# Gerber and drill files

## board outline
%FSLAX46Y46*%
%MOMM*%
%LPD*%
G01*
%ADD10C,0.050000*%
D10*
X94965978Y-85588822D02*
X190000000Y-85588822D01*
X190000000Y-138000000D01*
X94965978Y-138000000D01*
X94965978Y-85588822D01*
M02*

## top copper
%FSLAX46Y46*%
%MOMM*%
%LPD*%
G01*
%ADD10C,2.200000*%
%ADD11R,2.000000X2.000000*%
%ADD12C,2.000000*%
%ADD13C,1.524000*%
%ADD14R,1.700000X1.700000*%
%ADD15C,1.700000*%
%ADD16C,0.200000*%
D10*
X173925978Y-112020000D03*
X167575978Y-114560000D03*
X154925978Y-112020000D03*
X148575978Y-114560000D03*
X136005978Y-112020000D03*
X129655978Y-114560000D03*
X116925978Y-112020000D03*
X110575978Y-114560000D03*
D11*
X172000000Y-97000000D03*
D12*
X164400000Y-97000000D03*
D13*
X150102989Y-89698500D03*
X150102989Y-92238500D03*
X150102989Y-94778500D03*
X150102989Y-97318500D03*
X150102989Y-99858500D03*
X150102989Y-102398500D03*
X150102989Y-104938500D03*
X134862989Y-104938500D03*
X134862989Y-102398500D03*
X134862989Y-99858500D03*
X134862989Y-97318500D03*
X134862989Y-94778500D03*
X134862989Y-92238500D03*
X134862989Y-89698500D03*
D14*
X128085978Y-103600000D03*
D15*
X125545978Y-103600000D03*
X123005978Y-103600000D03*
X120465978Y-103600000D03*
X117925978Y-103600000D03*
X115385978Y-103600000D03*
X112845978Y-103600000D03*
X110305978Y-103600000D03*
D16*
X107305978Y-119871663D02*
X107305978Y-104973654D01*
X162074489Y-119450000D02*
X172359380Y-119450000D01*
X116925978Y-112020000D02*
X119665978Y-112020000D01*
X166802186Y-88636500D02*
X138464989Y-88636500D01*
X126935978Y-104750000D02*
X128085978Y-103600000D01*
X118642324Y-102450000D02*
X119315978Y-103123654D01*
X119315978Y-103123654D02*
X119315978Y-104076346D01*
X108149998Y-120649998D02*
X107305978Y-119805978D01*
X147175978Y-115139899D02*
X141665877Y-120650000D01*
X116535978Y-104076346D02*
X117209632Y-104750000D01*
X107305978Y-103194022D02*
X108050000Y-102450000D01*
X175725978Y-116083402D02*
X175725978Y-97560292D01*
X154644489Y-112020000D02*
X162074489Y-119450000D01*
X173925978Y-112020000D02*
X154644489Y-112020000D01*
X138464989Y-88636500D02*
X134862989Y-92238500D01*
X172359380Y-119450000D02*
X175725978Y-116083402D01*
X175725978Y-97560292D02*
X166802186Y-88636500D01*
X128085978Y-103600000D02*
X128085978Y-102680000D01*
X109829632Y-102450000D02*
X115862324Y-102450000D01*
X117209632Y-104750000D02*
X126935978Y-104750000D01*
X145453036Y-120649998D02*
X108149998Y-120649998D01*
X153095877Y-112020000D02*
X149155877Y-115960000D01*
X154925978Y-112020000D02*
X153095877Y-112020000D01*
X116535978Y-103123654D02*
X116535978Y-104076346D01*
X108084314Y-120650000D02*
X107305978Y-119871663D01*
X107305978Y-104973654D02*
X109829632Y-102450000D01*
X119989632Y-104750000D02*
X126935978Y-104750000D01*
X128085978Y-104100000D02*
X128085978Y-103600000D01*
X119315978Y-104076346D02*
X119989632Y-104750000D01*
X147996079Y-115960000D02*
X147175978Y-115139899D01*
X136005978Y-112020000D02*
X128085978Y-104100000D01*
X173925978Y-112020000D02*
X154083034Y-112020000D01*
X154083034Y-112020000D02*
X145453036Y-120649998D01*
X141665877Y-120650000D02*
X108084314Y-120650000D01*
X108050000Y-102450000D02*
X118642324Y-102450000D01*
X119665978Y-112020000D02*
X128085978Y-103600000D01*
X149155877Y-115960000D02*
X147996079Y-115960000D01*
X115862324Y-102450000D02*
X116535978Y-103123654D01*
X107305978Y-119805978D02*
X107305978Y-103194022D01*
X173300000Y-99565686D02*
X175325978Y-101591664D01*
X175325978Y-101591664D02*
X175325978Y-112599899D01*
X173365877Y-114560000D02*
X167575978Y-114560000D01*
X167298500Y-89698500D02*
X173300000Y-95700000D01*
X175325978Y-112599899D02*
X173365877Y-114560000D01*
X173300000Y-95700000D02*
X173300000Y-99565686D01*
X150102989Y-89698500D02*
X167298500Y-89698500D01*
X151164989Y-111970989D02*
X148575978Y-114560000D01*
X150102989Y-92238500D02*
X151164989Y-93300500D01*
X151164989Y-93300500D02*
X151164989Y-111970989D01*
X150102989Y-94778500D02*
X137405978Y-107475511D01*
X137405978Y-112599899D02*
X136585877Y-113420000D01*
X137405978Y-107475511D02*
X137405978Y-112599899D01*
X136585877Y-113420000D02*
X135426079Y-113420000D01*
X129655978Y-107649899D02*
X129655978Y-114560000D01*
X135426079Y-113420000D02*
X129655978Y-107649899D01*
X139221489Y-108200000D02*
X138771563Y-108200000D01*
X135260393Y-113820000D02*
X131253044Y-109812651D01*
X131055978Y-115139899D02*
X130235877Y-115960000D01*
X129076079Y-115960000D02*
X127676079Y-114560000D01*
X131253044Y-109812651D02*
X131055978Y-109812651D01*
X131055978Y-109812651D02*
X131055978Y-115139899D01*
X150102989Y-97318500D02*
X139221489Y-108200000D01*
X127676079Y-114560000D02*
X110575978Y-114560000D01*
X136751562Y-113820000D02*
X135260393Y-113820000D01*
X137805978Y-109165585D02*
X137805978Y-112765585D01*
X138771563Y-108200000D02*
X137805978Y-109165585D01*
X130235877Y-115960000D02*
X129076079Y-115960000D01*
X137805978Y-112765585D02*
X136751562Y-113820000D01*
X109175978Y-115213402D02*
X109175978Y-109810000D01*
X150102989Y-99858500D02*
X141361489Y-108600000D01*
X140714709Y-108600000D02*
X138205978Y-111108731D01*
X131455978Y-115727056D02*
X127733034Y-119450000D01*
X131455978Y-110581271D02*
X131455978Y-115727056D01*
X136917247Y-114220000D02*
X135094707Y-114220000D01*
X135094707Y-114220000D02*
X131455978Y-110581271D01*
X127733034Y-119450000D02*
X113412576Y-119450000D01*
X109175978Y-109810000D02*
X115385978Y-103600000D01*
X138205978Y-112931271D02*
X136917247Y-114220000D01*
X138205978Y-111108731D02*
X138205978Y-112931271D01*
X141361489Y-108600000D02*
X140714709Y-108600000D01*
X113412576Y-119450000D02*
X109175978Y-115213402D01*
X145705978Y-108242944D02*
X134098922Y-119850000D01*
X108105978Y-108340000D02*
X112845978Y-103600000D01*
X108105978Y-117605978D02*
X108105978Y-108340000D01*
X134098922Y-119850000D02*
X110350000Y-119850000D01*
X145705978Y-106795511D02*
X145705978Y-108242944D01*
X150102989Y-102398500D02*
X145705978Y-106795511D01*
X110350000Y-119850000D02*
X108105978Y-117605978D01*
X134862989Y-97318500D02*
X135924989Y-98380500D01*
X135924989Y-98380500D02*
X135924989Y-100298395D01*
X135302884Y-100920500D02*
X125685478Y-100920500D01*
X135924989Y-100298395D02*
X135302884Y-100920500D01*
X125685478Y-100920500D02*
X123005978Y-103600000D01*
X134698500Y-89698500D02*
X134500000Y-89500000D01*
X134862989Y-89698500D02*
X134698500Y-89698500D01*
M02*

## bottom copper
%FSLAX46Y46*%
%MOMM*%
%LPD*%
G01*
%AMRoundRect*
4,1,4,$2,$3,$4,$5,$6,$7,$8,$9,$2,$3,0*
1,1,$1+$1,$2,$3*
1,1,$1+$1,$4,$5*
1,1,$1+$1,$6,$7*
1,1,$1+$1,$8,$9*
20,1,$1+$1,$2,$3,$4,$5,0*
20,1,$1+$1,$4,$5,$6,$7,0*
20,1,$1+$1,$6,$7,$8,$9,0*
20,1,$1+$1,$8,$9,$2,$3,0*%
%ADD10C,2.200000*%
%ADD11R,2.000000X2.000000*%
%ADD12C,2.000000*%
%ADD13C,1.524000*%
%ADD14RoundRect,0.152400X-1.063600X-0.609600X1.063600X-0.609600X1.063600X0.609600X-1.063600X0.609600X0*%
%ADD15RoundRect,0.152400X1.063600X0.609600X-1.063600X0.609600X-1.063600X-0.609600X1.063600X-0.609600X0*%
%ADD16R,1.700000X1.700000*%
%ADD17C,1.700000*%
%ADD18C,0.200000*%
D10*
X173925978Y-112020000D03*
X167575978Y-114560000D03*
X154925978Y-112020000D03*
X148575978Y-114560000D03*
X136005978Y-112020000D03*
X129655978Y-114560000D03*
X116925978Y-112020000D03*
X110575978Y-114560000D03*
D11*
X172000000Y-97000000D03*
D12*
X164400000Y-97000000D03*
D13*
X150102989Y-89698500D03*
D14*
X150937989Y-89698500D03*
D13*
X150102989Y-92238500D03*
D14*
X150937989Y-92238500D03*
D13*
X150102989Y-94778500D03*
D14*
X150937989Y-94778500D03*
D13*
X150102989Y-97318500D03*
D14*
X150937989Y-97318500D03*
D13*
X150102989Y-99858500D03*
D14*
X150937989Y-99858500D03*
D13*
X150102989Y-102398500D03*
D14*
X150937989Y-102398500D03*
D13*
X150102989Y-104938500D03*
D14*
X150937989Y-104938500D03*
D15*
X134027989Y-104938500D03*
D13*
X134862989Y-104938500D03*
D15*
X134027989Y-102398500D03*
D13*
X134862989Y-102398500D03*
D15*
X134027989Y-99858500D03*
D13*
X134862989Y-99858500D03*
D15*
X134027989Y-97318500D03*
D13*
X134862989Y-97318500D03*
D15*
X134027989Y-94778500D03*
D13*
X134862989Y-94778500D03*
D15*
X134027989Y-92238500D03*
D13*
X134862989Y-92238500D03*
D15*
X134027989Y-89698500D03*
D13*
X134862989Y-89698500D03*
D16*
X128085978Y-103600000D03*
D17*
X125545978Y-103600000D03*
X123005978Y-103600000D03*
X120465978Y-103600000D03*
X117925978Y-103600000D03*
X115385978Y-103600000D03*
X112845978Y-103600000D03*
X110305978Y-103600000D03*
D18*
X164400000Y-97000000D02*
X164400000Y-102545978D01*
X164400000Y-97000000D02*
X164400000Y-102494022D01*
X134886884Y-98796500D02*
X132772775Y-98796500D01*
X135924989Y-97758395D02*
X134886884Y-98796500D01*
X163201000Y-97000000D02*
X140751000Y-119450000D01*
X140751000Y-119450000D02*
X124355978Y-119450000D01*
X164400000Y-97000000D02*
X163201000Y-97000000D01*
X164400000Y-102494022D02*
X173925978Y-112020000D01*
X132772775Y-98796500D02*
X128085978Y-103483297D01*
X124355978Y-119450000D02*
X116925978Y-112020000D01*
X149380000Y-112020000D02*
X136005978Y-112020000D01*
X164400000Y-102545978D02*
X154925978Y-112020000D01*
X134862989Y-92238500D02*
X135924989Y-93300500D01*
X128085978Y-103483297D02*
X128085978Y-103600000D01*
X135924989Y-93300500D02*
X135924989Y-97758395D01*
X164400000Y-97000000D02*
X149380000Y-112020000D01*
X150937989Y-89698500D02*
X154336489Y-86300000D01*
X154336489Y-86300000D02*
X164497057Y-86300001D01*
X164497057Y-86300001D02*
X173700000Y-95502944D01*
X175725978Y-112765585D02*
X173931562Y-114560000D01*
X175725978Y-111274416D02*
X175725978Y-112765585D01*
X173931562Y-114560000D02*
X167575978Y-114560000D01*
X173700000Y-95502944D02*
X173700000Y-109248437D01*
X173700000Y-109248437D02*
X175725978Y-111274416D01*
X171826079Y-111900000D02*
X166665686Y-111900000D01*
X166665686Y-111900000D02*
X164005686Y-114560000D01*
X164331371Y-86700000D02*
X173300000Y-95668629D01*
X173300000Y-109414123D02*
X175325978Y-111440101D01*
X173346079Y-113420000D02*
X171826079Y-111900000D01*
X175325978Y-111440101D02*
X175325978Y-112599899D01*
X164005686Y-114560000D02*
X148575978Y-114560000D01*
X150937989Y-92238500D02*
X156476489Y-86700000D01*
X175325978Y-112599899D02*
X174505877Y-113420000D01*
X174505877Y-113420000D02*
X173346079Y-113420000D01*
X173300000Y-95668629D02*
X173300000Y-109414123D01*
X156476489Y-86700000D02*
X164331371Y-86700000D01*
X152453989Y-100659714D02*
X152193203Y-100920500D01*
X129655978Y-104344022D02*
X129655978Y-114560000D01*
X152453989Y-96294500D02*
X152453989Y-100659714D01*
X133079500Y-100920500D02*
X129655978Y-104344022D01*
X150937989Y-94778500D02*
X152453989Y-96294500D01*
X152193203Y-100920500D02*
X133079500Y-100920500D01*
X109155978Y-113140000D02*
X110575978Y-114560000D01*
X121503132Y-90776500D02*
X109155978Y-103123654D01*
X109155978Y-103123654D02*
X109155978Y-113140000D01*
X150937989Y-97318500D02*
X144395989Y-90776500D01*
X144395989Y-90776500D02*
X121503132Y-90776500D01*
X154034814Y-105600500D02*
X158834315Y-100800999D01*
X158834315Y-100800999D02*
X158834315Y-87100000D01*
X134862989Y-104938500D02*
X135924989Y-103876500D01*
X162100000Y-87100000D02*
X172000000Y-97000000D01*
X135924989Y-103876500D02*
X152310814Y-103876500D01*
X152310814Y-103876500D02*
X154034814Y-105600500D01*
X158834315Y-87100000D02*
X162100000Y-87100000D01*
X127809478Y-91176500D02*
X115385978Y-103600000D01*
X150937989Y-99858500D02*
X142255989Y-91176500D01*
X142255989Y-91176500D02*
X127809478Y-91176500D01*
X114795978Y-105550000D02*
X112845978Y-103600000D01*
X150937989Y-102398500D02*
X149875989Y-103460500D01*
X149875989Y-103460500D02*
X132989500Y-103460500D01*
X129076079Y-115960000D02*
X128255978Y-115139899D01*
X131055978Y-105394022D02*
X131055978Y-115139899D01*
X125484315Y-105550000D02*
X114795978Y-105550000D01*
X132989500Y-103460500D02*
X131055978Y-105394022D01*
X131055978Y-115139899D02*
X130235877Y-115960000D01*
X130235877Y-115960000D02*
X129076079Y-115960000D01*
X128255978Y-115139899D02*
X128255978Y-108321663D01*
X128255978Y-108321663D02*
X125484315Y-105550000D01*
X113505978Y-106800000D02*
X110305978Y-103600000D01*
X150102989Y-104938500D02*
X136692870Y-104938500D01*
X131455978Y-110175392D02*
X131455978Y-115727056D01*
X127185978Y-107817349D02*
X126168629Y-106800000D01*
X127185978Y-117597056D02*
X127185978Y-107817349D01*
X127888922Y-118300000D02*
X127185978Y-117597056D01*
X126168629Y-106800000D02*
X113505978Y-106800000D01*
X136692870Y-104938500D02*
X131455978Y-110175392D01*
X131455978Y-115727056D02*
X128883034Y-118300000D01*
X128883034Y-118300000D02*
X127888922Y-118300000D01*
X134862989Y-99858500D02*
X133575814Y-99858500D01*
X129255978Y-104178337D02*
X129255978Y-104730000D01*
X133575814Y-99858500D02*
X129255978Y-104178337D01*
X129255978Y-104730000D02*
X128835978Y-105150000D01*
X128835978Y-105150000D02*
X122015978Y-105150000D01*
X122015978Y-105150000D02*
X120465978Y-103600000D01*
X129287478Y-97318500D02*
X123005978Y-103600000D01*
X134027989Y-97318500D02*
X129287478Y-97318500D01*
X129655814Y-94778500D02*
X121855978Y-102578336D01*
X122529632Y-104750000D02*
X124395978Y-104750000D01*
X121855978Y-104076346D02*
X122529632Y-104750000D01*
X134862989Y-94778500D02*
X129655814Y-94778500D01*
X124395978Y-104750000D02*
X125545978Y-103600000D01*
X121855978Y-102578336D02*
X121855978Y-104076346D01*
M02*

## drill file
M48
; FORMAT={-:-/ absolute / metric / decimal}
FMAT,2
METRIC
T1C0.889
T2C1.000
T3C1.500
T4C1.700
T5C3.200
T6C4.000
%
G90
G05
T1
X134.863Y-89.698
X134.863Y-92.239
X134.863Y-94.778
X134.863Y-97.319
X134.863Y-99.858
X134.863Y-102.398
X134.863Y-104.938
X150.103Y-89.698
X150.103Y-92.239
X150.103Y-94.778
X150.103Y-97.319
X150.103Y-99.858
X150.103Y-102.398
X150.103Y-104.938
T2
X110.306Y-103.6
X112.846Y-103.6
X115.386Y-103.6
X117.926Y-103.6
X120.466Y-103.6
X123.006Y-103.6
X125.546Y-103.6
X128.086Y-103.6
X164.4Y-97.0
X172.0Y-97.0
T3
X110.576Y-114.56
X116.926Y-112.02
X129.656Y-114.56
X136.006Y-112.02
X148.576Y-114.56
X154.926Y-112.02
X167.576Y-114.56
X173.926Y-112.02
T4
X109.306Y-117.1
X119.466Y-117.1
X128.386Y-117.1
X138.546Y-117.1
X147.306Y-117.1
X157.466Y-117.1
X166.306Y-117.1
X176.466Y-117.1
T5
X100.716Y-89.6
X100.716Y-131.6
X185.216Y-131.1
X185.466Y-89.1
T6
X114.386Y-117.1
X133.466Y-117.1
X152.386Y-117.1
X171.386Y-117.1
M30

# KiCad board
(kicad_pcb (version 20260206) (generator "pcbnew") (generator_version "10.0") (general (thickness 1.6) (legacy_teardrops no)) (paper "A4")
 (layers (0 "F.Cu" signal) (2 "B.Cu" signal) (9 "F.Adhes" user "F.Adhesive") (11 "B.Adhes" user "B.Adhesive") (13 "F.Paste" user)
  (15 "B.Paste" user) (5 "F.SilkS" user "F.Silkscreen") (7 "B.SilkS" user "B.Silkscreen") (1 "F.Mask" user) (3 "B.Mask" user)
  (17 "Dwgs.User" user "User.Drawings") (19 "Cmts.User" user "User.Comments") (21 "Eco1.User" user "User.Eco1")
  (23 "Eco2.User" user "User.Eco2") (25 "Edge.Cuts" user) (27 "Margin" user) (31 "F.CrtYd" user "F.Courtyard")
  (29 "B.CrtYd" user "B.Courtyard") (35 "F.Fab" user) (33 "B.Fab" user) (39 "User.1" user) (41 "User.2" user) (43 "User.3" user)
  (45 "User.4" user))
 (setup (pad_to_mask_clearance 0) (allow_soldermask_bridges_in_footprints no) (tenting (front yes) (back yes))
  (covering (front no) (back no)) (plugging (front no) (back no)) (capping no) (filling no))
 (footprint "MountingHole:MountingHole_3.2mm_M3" (layer "F.Cu") (at 185.215978 131.1)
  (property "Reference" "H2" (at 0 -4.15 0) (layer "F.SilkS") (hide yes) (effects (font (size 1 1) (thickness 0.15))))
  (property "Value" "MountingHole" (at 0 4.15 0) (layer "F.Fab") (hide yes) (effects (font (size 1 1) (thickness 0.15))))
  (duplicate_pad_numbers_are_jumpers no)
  (pad "" np_thru_hole circle (at 0 0) (size 3.2 3.2) (drill 3.2) (layers "*.Cu" "*.Mask")))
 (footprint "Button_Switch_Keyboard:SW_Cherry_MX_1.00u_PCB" (layer "F.Cu") (at 173.925978 112.02)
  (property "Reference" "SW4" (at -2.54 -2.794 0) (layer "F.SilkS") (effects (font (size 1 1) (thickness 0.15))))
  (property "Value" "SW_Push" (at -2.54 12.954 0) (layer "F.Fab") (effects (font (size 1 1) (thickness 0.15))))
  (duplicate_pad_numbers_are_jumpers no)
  (pad "" np_thru_hole circle (at -7.62 5.08) (size 1.7 1.7) (drill 1.7) (layers "*.Cu" "*.Mask"))
  (pad "" np_thru_hole circle (at -2.54 5.08) (size 4 4) (drill 4) (layers "*.Cu" "*.Mask"))
  (pad "" np_thru_hole circle (at 2.54 5.08) (size 1.7 1.7) (drill 1.7) (layers "*.Cu" "*.Mask"))
  (pad "1" thru_hole circle (at 0 0) (size 2.2 2.2) (drill 1.5) (layers "*.Cu" "*.Mask") (remove_unused_layers no) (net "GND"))
  (pad "2" thru_hole circle (at -6.35 2.54) (size 2.2 2.2) (drill 1.5) (layers "*.Cu" "*.Mask") (remove_unused_layers no)
   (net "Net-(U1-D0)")))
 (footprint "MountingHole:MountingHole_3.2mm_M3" (layer "F.Cu") (at 100.715978 131.6)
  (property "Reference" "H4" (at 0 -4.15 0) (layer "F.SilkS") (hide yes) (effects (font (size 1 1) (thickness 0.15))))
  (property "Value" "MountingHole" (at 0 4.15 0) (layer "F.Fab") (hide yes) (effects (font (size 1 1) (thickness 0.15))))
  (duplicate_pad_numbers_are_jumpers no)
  (pad "" np_thru_hole circle (at 0 0) (size 3.2 3.2) (drill 3.2) (layers "*.Cu" "*.Mask")))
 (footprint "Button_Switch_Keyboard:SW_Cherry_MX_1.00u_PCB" (layer "F.Cu") (at 154.925978 112.02)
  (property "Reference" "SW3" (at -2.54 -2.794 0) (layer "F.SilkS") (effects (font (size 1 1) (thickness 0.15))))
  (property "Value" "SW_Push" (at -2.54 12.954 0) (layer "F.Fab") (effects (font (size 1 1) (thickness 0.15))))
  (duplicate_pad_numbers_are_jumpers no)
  (pad "" np_thru_hole circle (at -7.62 5.08) (size 1.7 1.7) (drill 1.7) (layers "*.Cu" "*.Mask"))
  (pad "" np_thru_hole circle (at -2.54 5.08) (size 4 4) (drill 4) (layers "*.Cu" "*.Mask"))
  (pad "" np_thru_hole circle (at 2.54 5.08) (size 1.7 1.7) (drill 1.7) (layers "*.Cu" "*.Mask"))
  (pad "1" thru_hole circle (at 0 0) (size 2.2 2.2) (drill 1.5) (layers "*.Cu" "*.Mask") (remove_unused_layers no) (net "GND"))
  (pad "2" thru_hole circle (at -6.35 2.54) (size 2.2 2.2) (drill 1.5) (layers "*.Cu" "*.Mask") (remove_unused_layers no)
   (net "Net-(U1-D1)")))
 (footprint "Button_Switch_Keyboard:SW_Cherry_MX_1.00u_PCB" (layer "F.Cu") (at 136.005978 112.02)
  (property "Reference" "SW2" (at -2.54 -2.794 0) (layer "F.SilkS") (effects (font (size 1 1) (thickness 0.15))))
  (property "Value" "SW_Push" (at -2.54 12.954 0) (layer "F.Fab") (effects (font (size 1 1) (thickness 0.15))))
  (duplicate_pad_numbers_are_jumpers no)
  (pad "" np_thru_hole circle (at -7.62 5.08) (size 1.7 1.7) (drill 1.7) (layers "*.Cu" "*.Mask"))
  (pad "" np_thru_hole circle (at -2.54 5.08) (size 4 4) (drill 4) (layers "*.Cu" "*.Mask"))
  (pad "" np_thru_hole circle (at 2.54 5.08) (size 1.7 1.7) (drill 1.7) (layers "*.Cu" "*.Mask"))
  (pad "1" thru_hole circle (at 0 0) (size 2.2 2.2) (drill 1.5) (layers "*.Cu" "*.Mask") (remove_unused_layers no) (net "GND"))
  (pad "2" thru_hole circle (at -6.35 2.54) (size 2.2 2.2) (drill 1.5) (layers "*.Cu" "*.Mask") (remove_unused_layers no)
   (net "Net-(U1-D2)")))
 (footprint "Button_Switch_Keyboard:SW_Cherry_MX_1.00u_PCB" (layer "F.Cu") (at 116.925978 112.02)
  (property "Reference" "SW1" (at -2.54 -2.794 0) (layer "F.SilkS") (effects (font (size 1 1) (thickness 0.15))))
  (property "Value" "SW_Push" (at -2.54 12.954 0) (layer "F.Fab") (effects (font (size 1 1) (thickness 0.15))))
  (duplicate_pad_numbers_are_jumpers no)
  (pad "" np_thru_hole circle (at -7.62 5.08) (size 1.7 1.7) (drill 1.7) (layers "*.Cu" "*.Mask"))
  (pad "" np_thru_hole circle (at -2.54 5.08) (size 4 4) (drill 4) (layers "*.Cu" "*.Mask"))
  (pad "" np_thru_hole circle (at 2.54 5.08) (size 1.7 1.7) (drill 1.7) (layers "*.Cu" "*.Mask"))
  (pad "1" thru_hole circle (at 0 0) (size 2.2 2.2) (drill 1.5) (layers "*.Cu" "*.Mask") (remove_unused_layers no) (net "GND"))
  (pad "2" thru_hole circle (at -6.35 2.54) (size 2.2 2.2) (drill 1.5) (layers "*.Cu" "*.Mask") (remove_unused_layers no)
   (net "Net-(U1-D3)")))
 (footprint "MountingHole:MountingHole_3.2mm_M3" (layer "F.Cu") (at 100.715978 89.6)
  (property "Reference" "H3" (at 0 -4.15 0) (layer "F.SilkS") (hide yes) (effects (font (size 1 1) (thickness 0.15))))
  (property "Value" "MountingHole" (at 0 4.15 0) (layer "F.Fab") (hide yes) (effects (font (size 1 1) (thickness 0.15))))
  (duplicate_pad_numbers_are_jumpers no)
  (pad "" np_thru_hole circle (at 0 0) (size 3.2 3.2) (drill 3.2) (layers "*.Cu" "*.Mask")))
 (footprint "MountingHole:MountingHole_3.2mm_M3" (layer "F.Cu") (at 185.465978 89.1)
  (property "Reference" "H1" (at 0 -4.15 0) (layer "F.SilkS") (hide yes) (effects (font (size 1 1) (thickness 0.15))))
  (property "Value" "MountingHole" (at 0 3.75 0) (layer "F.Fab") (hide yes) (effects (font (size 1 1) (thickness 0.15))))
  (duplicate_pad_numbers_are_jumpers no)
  (pad "" np_thru_hole circle (at 0 0) (size 3.2 3.2) (drill 3.2) (layers "*.Cu" "*.Mask")))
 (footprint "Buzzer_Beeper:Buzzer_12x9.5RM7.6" (layer "B.Cu") (at 172 97 180)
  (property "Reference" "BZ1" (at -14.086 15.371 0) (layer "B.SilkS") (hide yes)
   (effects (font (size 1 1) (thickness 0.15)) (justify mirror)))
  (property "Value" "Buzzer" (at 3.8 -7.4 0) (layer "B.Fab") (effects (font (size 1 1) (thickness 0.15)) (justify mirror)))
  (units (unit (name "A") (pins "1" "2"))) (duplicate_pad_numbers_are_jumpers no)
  (pad "1" thru_hole rect (at 0 0 180) (size 2 2) (drill 1) (layers "*.Cu" "*.Mask") (remove_unused_layers no) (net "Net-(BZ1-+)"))
  (pad "2" thru_hole circle (at 7.6 0 180) (size 2 2) (drill 1) (layers "*.Cu" "*.Mask") (remove_unused_layers no) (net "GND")))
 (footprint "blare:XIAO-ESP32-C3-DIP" (layer "B.Cu") (at 142.482989 97.3185 90)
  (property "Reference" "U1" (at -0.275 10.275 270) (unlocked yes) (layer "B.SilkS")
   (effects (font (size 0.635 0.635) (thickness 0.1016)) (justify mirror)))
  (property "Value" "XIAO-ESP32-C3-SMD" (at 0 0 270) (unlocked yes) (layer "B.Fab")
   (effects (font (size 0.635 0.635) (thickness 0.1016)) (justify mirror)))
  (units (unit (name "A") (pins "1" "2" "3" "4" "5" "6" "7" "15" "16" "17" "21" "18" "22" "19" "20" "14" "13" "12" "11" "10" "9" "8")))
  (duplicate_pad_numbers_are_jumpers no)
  (pad "1" thru_hole circle (at 7.62 7.62) (size 1.524 1.524) (drill 0.889) (layers "*.Cu" "*.Mask") (remove_unused_layers no)
   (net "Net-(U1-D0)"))
  (pad "1" smd roundrect (at 7.62 8.455) (size 2.432 1.524) (layers "B.Cu" "B.Mask") (roundrect_rratio 0.1) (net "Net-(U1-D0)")
   (thermal_bridge_angle 45))
  (pad "2" thru_hole circle (at 5.08 7.62) (size 1.524 1.524) (drill 0.889) (layers "*.Cu" "*.Mask") (remove_unused_layers no)
   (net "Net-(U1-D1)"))
  (pad "2" smd roundrect (at 5.08 8.455) (size 2.432 1.524) (layers "B.Cu" "B.Mask") (roundrect_rratio 0.1) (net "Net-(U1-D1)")
   (thermal_bridge_angle 45))
  (pad "3" thru_hole circle (at 2.54 7.62) (size 1.524 1.524) (drill 0.889) (layers "*.Cu" "*.Mask") (remove_unused_layers no)
   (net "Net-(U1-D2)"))
  (pad "3" smd roundrect (at 2.54 8.455) (size 2.432 1.524) (layers "B.Cu" "B.Mask") (roundrect_rratio 0.1) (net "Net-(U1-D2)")
   (thermal_bridge_angle 45))
  (pad "4" thru_hole circle (at 0 7.62) (size 1.524 1.524) (drill 0.889) (layers "*.Cu" "*.Mask") (remove_unused_layers no)
   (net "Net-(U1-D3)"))
  (pad "4" smd roundrect (at 0 8.455) (size 2.432 1.524) (layers "B.Cu" "B.Mask") (roundrect_rratio 0.1) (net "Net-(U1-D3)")
   (thermal_bridge_angle 45))
  (pad "5" thru_hole circle (at -2.54 7.62) (size 1.524 1.524) (drill 0.889) (layers "*.Cu" "*.Mask") (remove_unused_layers no) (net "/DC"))
  (pad "5" smd roundrect (at -2.54 8.455) (size 2.432 1.524) (layers "B.Cu" "B.Mask") (roundrect_rratio 0.1) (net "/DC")
   (thermal_bridge_angle 45))
  (pad "6" thru_hole circle (at -5.08 7.62) (size 1.524 1.524) (drill 0.889) (layers "*.Cu" "*.Mask") (remove_unused_layers no) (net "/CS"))
  (pad "6" smd roundrect (at -5.08 8.455) (size 2.432 1.524) (layers "B.Cu" "B.Mask") (roundrect_rratio 0.1) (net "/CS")
   (thermal_bridge_angle 45))
  (pad "7" thru_hole circle (at -7.62 7.62) (size 1.524 1.524) (drill 0.889) (layers "*.Cu" "*.Mask") (remove_unused_layers no) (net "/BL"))
  (pad "7" smd roundrect (at -7.62 8.455) (size 2.432 1.524) (layers "B.Cu" "B.Mask") (roundrect_rratio 0.1) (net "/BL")
   (thermal_bridge_angle 45))
  (pad "8" smd roundrect (at -7.62 -8.455 180) (size 2.432 1.524) (layers "B.Cu" "B.Mask") (roundrect_rratio 0.1) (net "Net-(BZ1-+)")
   (thermal_bridge_angle 45))
  (pad "8" thru_hole circle (at -7.62 -7.62 180) (size 1.524 1.524) (drill 0.889) (layers "*.Cu" "*.Mask") (remove_unused_layers no)
   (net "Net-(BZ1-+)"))
  (pad "9" smd roundrect (at -5.08 -8.455 180) (size 2.432 1.524) (layers "B.Cu" "B.Mask") (roundrect_rratio 0.1) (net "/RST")
   (thermal_bridge_angle 45))
  (pad "9" thru_hole circle (at -5.08 -7.62 180) (size 1.524 1.524) (drill 0.889) (layers "*.Cu" "*.Mask") (remove_unused_layers no)
   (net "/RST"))
  (pad "10" smd roundrect (at -2.54 -8.455 180) (size 2.432 1.524) (layers "B.Cu" "B.Mask") (roundrect_rratio 0.1) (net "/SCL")
   (thermal_bridge_angle 45))
  (pad "10" thru_hole circle (at -2.54 -7.62 180) (size 1.524 1.524) (drill 0.889) (layers "*.Cu" "*.Mask") (remove_unused_layers no)
   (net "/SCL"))
  (pad "11" smd roundrect (at 0 -8.455 180) (size 2.432 1.524) (layers "B.Cu" "B.Mask") (roundrect_rratio 0.1) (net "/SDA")
   (thermal_bridge_angle 45))
  (pad "11" thru_hole circle (at 0 -7.62 180) (size 1.524 1.524) (drill 0.889) (layers "*.Cu" "*.Mask") (remove_unused_layers no)
   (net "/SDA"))
  (pad "12" smd roundrect (at 2.54 -8.455 180) (size 2.432 1.524) (layers "B.Cu" "B.Mask") (roundrect_rratio 0.1) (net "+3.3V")
   (thermal_bridge_angle 45))
  (pad "12" thru_hole circle (at 2.54 -7.62 180) (size 1.524 1.524) (drill 0.889) (layers "*.Cu" "*.Mask") (remove_unused_layers no)
   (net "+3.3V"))
  (pad "13" smd roundrect (at 5.08 -8.455 180) (size 2.432 1.524) (layers "B.Cu" "B.Mask") (roundrect_rratio 0.1) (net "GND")
   (thermal_bridge_angle 45))
  (pad "13" thru_hole circle (at 5.08 -7.62 180) (size 1.524 1.524) (drill 0.889) (layers "*.Cu" "*.Mask") (remove_unused_layers no)
   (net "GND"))
  (pad "14" smd roundrect (at 7.62 -8.455 180) (size 2.432 1.524) (layers "B.Cu" "B.Mask") (roundrect_rratio 0.1)
   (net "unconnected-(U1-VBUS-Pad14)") (thermal_bridge_angle 45))
  (pad "14" thru_hole circle (at 7.62 -7.62 180) (size 1.524 1.524) (drill 0.889) (layers "*.Cu" "*.Mask") (remove_unused_layers no)
   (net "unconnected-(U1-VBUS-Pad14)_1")))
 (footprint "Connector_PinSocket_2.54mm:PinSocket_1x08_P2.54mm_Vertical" (layer "B.Cu") (at 128.085978 103.6 90)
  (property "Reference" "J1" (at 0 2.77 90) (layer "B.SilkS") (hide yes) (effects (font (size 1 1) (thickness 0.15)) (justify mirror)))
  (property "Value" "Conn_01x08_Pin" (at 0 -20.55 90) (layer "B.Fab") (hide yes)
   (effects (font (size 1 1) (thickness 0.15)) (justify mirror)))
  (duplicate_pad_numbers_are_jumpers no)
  (pad "1" thru_hole rect (at 0 0 90) (size 1.7 1.7) (drill 1) (layers "*.Cu" "*.Mask") (remove_unused_layers no) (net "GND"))
  (pad "2" thru_hole circle (at 0 -2.54 90) (size 1.7 1.7) (drill 1) (layers "*.Cu" "*.Mask") (remove_unused_layers no) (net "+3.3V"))
  (pad "3" thru_hole circle (at 0 -5.08 90) (size 1.7 1.7) (drill 1) (layers "*.Cu" "*.Mask") (remove_unused_layers no) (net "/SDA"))
  (pad "4" thru_hole circle (at 0 -7.62 90) (size 1.7 1.7) (drill 1) (layers "*.Cu" "*.Mask") (remove_unused_layers no) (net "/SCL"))
  (pad "5" thru_hole circle (at 0 -10.16 90) (size 1.7 1.7) (drill 1) (layers "*.Cu" "*.Mask") (remove_unused_layers no) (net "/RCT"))
  (pad "6" thru_hole circle (at 0 -12.7 90) (size 1.7 1.7) (drill 1) (layers "*.Cu" "*.Mask") (remove_unused_layers no) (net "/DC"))
  (pad "7" thru_hole circle (at 0 -15.24 90) (size 1.7 1.7) (drill 1) (layers "*.Cu" "*.Mask") (remove_unused_layers no) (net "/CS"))
  (pad "8" thru_hole circle (at 0 -17.78 90) (size 1.7 1.7) (drill 1) (layers "*.Cu" "*.Mask") (remove_unused_layers no) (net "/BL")))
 (gr_rect (start 94.965978 85.588822) (end 190 138) (stroke (width 0.05) (type default)) (fill no) (layer "Edge.Cuts"))
 (segment (start 107.305978 119.871663) (end 107.305978 104.973654) (width 0.2) (layer "F.Cu") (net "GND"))
 (segment (start 162.074489 119.45) (end 172.35938 119.45) (width 0.2) (layer "F.Cu") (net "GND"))
 (segment (start 116.925978 112.02) (end 119.665978 112.02) (width 0.2) (layer "F.Cu") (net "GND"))
 (segment (start 166.802186 88.6365) (end 138.464989 88.6365) (width 0.2) (layer "F.Cu") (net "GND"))
 (segment (start 126.935978 104.75) (end 128.085978 103.6) (width 0.2) (layer "F.Cu") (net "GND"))
 (segment (start 118.642324 102.45) (end 119.315978 103.123654) (width 0.2) (layer "F.Cu") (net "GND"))
 (segment (start 119.315978 103.123654) (end 119.315978 104.076346) (width 0.2) (layer "F.Cu") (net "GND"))
 (segment (start 108.149998 120.649998) (end 107.305978 119.805978) (width 0.2) (layer "F.Cu") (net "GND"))
 (segment (start 147.175978 115.139899) (end 141.665877 120.65) (width 0.2) (layer "F.Cu") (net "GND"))
 (segment (start 116.535978 104.076346) (end 117.209632 104.75) (width 0.2) (layer "F.Cu") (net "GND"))
 (segment (start 107.305978 103.194022) (end 108.05 102.45) (width 0.2) (layer "F.Cu") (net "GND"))
 (segment (start 175.725978 116.083402) (end 175.725978 97.560292) (width 0.2) (layer "F.Cu") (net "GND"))
 (segment (start 154.644489 112.02) (end 162.074489 119.45) (width 0.2) (layer "F.Cu") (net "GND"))
 (segment (start 173.925978 112.02) (end 154.644489 112.02) (width 0.2) (layer "F.Cu") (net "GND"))
 (segment (start 138.464989 88.6365) (end 134.862989 92.2385) (width 0.2) (layer "F.Cu") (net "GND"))
 (segment (start 172.35938 119.45) (end 175.725978 116.083402) (width 0.2) (layer "F.Cu") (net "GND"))
 (segment (start 175.725978 97.560292) (end 166.802186 88.6365) (width 0.2) (layer "F.Cu") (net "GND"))
 (segment (start 128.085978 103.6) (end 128.085978 102.68) (width 0.2) (layer "F.Cu") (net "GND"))
 (segment (start 109.829632 102.45) (end 115.862324 102.45) (width 0.2) (layer "F.Cu") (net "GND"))
 (segment (start 117.209632 104.75) (end 126.935978 104.75) (width 0.2) (layer "F.Cu") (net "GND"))
 (segment (start 145.453036 120.649998) (end 108.149998 120.649998) (width 0.2) (layer "F.Cu") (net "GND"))
 (segment (start 153.095877 112.02) (end 149.155877 115.96) (width 0.2) (layer "F.Cu") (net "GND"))
 (segment (start 154.925978 112.02) (end 153.095877 112.02) (width 0.2) (layer "F.Cu") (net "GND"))
 (segment (start 116.535978 103.123654) (end 116.535978 104.076346) (width 0.2) (layer "F.Cu") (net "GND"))
 (segment (start 108.084314 120.65) (end 107.305978 119.871663) (width 0.2) (layer "F.Cu") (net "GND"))
 (segment (start 107.305978 104.973654) (end 109.829632 102.45) (width 0.2) (layer "F.Cu") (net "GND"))
 (segment (start 119.989632 104.75) (end 126.935978 104.75) (width 0.2) (layer "F.Cu") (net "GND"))
 (segment (start 128.085978 104.1) (end 128.085978 103.6) (width 0.2) (layer "F.Cu") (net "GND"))
 (segment (start 119.315978 104.076346) (end 119.989632 104.75) (width 0.2) (layer "F.Cu") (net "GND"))
 (segment (start 147.996079 115.96) (end 147.175978 115.139899) (width 0.2) (layer "F.Cu") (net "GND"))
 (segment (start 136.005978 112.02) (end 128.085978 104.1) (width 0.2) (layer "F.Cu") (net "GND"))
 (segment (start 173.925978 112.02) (end 154.083034 112.02) (width 0.2) (layer "F.Cu") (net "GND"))
 (segment (start 154.083034 112.02) (end 145.453036 120.649998) (width 0.2) (layer "F.Cu") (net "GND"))
 (segment (start 141.665877 120.65) (end 108.084314 120.65) (width 0.2) (layer "F.Cu") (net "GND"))
 (segment (start 108.05 102.45) (end 118.642324 102.45) (width 0.2) (layer "F.Cu") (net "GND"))
 (segment (start 119.665978 112.02) (end 128.085978 103.6) (width 0.2) (layer "F.Cu") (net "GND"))
 (segment (start 149.155877 115.96) (end 147.996079 115.96) (width 0.2) (layer "F.Cu") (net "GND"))
 (segment (start 115.862324 102.45) (end 116.535978 103.123654) (width 0.2) (layer "F.Cu") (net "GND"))
 (segment (start 107.305978 119.805978) (end 107.305978 103.194022) (width 0.2) (layer "F.Cu") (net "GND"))
 (segment (start 164.4 97) (end 164.4 102.545978) (width 0.2) (layer "B.Cu") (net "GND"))
 (segment (start 164.4 97) (end 164.4 102.494022) (width 0.2) (layer "B.Cu") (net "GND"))
 (segment (start 134.886884 98.7965) (end 132.772775 98.7965) (width 0.2) (layer "B.Cu") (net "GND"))
 (segment (start 135.924989 97.758395) (end 134.886884 98.7965) (width 0.2) (layer "B.Cu") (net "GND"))
 (segment (start 163.201 97) (end 140.751 119.45) (width 0.2) (layer "B.Cu") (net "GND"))
 (segment (start 140.751 119.45) (end 124.355978 119.45) (width 0.2) (layer "B.Cu") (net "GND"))
 (segment (start 164.4 97) (end 163.201 97) (width 0.2) (layer "B.Cu") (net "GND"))
 (segment (start 164.4 102.494022) (end 173.925978 112.02) (width 0.2) (layer "B.Cu") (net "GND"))
 (segment (start 132.772775 98.7965) (end 128.085978 103.483297) (width 0.2) (layer "B.Cu") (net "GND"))
 (segment (start 124.355978 119.45) (end 116.925978 112.02) (width 0.2) (layer "B.Cu") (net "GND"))
 (segment (start 149.38 112.02) (end 136.005978 112.02) (width 0.2) (layer "B.Cu") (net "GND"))
 (segment (start 164.4 102.545978) (end 154.925978 112.02) (width 0.2) (layer "B.Cu") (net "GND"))
 (segment (start 134.862989 92.2385) (end 135.924989 93.3005) (width 0.2) (layer "B.Cu") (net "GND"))
 (segment (start 128.085978 103.483297) (end 128.085978 103.6) (width 0.2) (layer "B.Cu") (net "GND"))
 (segment (start 135.924989 93.3005) (end 135.924989 97.758395) (width 0.2) (layer "B.Cu") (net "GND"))
 (segment (start 164.4 97) (end 149.38 112.02) (width 0.2) (layer "B.Cu") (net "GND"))
 (segment (start 173.3 99.565686) (end 175.325978 101.591664) (width 0.2) (layer "F.Cu") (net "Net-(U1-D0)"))
 (segment (start 175.325978 101.591664) (end 175.325978 112.599899) (width 0.2) (layer "F.Cu") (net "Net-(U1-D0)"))
 (segment (start 173.365877 114.56) (end 167.575978 114.56) (width 0.2) (layer "F.Cu") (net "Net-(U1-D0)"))
 (segment (start 167.2985 89.6985) (end 173.3 95.7) (width 0.2) (layer "F.Cu") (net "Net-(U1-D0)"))
 (segment (start 175.325978 112.599899) (end 173.365877 114.56) (width 0.2) (layer "F.Cu") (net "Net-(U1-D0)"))
 (segment (start 173.3 95.7) (end 173.3 99.565686) (width 0.2) (layer "F.Cu") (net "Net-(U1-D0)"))
 (segment (start 150.102989 89.6985) (end 167.2985 89.6985) (width 0.2) (layer "F.Cu") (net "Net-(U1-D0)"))
 (segment (start 150.937989 89.6985) (end 154.336489 86.3) (width 0.2) (layer "B.Cu") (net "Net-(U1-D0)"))
 (segment (start 154.336489 86.3) (end 164.497057 86.300001) (width 0.2) (layer "B.Cu") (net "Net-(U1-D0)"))
 (segment (start 164.497057 86.300001) (end 173.7 95.502944) (width 0.2) (layer "B.Cu") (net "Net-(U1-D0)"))
 (segment (start 175.725978 112.765585) (end 173.931562 114.56) (width 0.2) (layer "B.Cu") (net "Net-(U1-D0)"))
 (segment (start 175.725978 111.274416) (end 175.725978 112.765585) (width 0.2) (layer "B.Cu") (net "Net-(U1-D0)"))
 (segment (start 173.931562 114.56) (end 167.575978 114.56) (width 0.2) (layer "B.Cu") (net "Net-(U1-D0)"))
 (segment (start 173.7 95.502944) (end 173.7 109.248437) (width 0.2) (layer "B.Cu") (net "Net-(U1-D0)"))
 (segment (start 173.7 109.248437) (end 175.725978 111.274416) (width 0.2) (layer "B.Cu") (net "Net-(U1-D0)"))
 (segment (start 151.164989 111.970989) (end 148.575978 114.56) (width 0.2) (layer "F.Cu") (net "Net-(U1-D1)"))
 (segment (start 150.102989 92.2385) (end 151.164989 93.3005) (width 0.2) (layer "F.Cu") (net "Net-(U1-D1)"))
 (segment (start 151.164989 93.3005) (end 151.164989 111.970989) (width 0.2) (layer "F.Cu") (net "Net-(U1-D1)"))
 (segment (start 171.826079 111.9) (end 166.665686 111.9) (width 0.2) (layer "B.Cu") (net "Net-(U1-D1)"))
 (segment (start 166.665686 111.9) (end 164.005686 114.56) (width 0.2) (layer "B.Cu") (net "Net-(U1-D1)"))
 (segment (start 164.331371 86.7) (end 173.3 95.668629) (width 0.2) (layer "B.Cu") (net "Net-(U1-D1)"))
 (segment (start 173.3 109.414123) (end 175.325978 111.440101) (width 0.2) (layer "B.Cu") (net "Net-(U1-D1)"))
 (segment (start 173.346079 113.42) (end 171.826079 111.9) (width 0.2) (layer "B.Cu") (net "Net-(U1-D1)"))
 (segment (start 175.325978 111.440101) (end 175.325978 112.599899) (width 0.2) (layer "B.Cu") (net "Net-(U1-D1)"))
 (segment (start 164.005686 114.56) (end 148.575978 114.56) (width 0.2) (layer "B.Cu") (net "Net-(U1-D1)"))
 (segment (start 150.937989 92.2385) (end 156.476489 86.7) (width 0.2) (layer "B.Cu") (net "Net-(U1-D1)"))
 (segment (start 175.325978 112.599899) (end 174.505877 113.42) (width 0.2) (layer "B.Cu") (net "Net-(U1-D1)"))
 (segment (start 174.505877 113.42) (end 173.346079 113.42) (width 0.2) (layer "B.Cu") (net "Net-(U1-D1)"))
 (segment (start 173.3 95.668629) (end 173.3 109.414123) (width 0.2) (layer "B.Cu") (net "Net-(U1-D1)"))
 (segment (start 156.476489 86.7) (end 164.331371 86.7) (width 0.2) (layer "B.Cu") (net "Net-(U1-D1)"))
 (segment (start 150.102989 94.7785) (end 137.405978 107.475511) (width 0.2) (layer "F.Cu") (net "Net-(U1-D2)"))
 (segment (start 137.405978 112.599899) (end 136.585877 113.42) (width 0.2) (layer "F.Cu") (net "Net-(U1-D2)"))
 (segment (start 137.405978 107.475511) (end 137.405978 112.599899) (width 0.2) (layer "F.Cu") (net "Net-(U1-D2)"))
 (segment (start 136.585877 113.42) (end 135.426079 113.42) (width 0.2) (layer "F.Cu") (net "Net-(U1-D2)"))
 (segment (start 129.655978 107.649899) (end 129.655978 114.56) (width 0.2) (layer "F.Cu") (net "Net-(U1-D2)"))
 (segment (start 135.426079 113.42) (end 129.655978 107.649899) (width 0.2) (layer "F.Cu") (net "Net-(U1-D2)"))
 (segment (start 152.453989 100.659714) (end 152.193203 100.9205) (width 0.2) (layer "B.Cu") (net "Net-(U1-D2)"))
 (segment (start 129.655978 104.344022) (end 129.655978 114.56) (width 0.2) (layer "B.Cu") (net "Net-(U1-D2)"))
 (segment (start 152.453989 96.2945) (end 152.453989 100.659714) (width 0.2) (layer "B.Cu") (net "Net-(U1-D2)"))
 (segment (start 133.0795 100.9205) (end 129.655978 104.344022) (width 0.2) (layer "B.Cu") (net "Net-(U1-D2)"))
 (segment (start 150.937989 94.7785) (end 152.453989 96.2945) (width 0.2) (layer "B.Cu") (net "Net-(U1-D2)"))
 (segment (start 152.193203 100.9205) (end 133.0795 100.9205) (width 0.2) (layer "B.Cu") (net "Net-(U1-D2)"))
 (segment (start 139.221489 108.2) (end 138.771563 108.2) (width 0.2) (layer "F.Cu") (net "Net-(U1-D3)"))
 (segment (start 135.260393 113.82) (end 131.253044 109.812651) (width 0.2) (layer "F.Cu") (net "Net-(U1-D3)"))
 (segment (start 131.055978 115.139899) (end 130.235877 115.96) (width 0.2) (layer "F.Cu") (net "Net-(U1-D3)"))
 (segment (start 129.076079 115.96) (end 127.676079 114.56) (width 0.2) (layer "F.Cu") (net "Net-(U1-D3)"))
 (segment (start 131.253044 109.812651) (end 131.055978 109.812651) (width 0.2) (layer "F.Cu") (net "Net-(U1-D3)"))
 (segment (start 131.055978 109.812651) (end 131.055978 115.139899) (width 0.2) (layer "F.Cu") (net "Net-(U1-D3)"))
 (segment (start 150.102989 97.3185) (end 139.221489 108.2) (width 0.2) (layer "F.Cu") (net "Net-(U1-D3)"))
 (segment (start 127.676079 114.56) (end 110.575978 114.56) (width 0.2) (layer "F.Cu") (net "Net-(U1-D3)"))
 (segment (start 136.751562 113.82) (end 135.260393 113.82) (width 0.2) (layer "F.Cu") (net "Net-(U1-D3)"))
 (segment (start 137.805978 109.165585) (end 137.805978 112.765585) (width 0.2) (layer "F.Cu") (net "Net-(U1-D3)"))
 (segment (start 138.771563 108.2) (end 137.805978 109.165585) (width 0.2) (layer "F.Cu") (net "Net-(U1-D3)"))
 (segment (start 130.235877 115.96) (end 129.076079 115.96) (width 0.2) (layer "F.Cu") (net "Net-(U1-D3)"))
 (segment (start 137.805978 112.765585) (end 136.751562 113.82) (width 0.2) (layer "F.Cu") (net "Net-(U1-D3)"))
 (segment (start 109.155978 113.14) (end 110.575978 114.56) (width 0.2) (layer "B.Cu") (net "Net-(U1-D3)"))
 (segment (start 121.503132 90.7765) (end 109.155978 103.123654) (width 0.2) (layer "B.Cu") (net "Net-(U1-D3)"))
 (segment (start 109.155978 103.123654) (end 109.155978 113.14) (width 0.2) (layer "B.Cu") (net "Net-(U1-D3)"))
 (segment (start 150.937989 97.3185) (end 144.395989 90.7765) (width 0.2) (layer "B.Cu") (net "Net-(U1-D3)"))
 (segment (start 144.395989 90.7765) (end 121.503132 90.7765) (width 0.2) (layer "B.Cu") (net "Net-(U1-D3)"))
 (segment (start 154.034814 105.6005) (end 158.834315 100.800999) (width 0.2) (layer "B.Cu") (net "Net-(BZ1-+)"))
 (segment (start 158.834315 100.800999) (end 158.834315 87.1) (width 0.2) (layer "B.Cu") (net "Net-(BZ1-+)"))
 (segment (start 134.862989 104.9385) (end 135.924989 103.8765) (width 0.2) (layer "B.Cu") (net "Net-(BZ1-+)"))
 (segment (start 162.1 87.1) (end 172 97) (width 0.2) (layer "B.Cu") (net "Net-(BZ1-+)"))
 (segment (start 135.924989 103.8765) (end 152.310814 103.8765) (width 0.2) (layer "B.Cu") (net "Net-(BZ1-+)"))
 (segment (start 152.310814 103.8765) (end 154.034814 105.6005) (width 0.2) (layer "B.Cu") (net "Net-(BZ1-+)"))
 (segment (start 158.834315 87.1) (end 162.1 87.1) (width 0.2) (layer "B.Cu") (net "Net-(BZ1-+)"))
 (segment (start 109.175978 115.213402) (end 109.175978 109.81) (width 0.2) (layer "F.Cu") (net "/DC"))
 (segment (start 150.102989 99.8585) (end 141.361489 108.6) (width 0.2) (layer "F.Cu") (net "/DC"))
 (segment (start 140.714709 108.6) (end 138.205978 111.108731) (width 0.2) (layer "F.Cu") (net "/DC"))
 (segment (start 131.455978 115.727056) (end 127.733034 119.45) (width 0.2) (layer "F.Cu") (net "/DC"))
 (segment (start 131.455978 110.581271) (end 131.455978 115.727056) (width 0.2) (layer "F.Cu") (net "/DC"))
 (segment (start 136.917247 114.22) (end 135.094707 114.22) (width 0.2) (layer "F.Cu") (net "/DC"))
 (segment (start 135.094707 114.22) (end 131.455978 110.581271) (width 0.2) (layer "F.Cu") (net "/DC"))
 (segment (start 127.733034 119.45) (end 113.412576 119.45) (width 0.2) (layer "F.Cu") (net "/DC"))
 (segment (start 109.175978 109.81) (end 115.385978 103.6) (width 0.2) (layer "F.Cu") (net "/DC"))
 (segment (start 138.205978 112.931271) (end 136.917247 114.22) (width 0.2) (layer "F.Cu") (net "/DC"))
 (segment (start 138.205978 111.108731) (end 138.205978 112.931271) (width 0.2) (layer "F.Cu") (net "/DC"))
 (segment (start 141.361489 108.6) (end 140.714709 108.6) (width 0.2) (layer "F.Cu") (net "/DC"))
 (segment (start 113.412576 119.45) (end 109.175978 115.213402) (width 0.2) (layer "F.Cu") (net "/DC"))
 (segment (start 127.809478 91.1765) (end 115.385978 103.6) (width 0.2) (layer "B.Cu") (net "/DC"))
 (segment (start 150.937989 99.8585) (end 142.255989 91.1765) (width 0.2) (layer "B.Cu") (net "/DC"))
 (segment (start 142.255989 91.1765) (end 127.809478 91.1765) (width 0.2) (layer "B.Cu") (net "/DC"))
 (segment (start 145.705978 108.242944) (end 134.098922 119.85) (width 0.2) (layer "F.Cu") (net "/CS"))
 (segment (start 108.105978 108.34) (end 112.845978 103.6) (width 0.2) (layer "F.Cu") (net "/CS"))
 (segment (start 108.105978 117.605978) (end 108.105978 108.34) (width 0.2) (layer "F.Cu") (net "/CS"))
 (segment (start 134.098922 119.85) (end 110.35 119.85) (width 0.2) (layer "F.Cu") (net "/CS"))
 (segment (start 145.705978 106.795511) (end 145.705978 108.242944) (width 0.2) (layer "F.Cu") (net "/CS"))
 (segment (start 150.102989 102.3985) (end 145.705978 106.795511) (width 0.2) (layer "F.Cu") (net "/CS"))
 (segment (start 110.35 119.85) (end 108.105978 117.605978) (width 0.2) (layer "F.Cu") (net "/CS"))
 (segment (start 114.795978 105.55) (end 112.845978 103.6) (width 0.2) (layer "B.Cu") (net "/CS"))
 (segment (start 150.937989 102.3985) (end 149.875989 103.4605) (width 0.2) (layer "B.Cu") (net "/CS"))
 (segment (start 149.875989 103.4605) (end 132.9895 103.4605) (width 0.2) (layer "B.Cu") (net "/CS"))
 (segment (start 129.076079 115.96) (end 128.255978 115.139899) (width 0.2) (layer "B.Cu") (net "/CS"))
 (segment (start 131.055978 105.394022) (end 131.055978 115.139899) (width 0.2) (layer "B.Cu") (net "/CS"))
 (segment (start 125.484315 105.55) (end 114.795978 105.55) (width 0.2) (layer "B.Cu") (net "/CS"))
 (segment (start 132.9895 103.4605) (end 131.055978 105.394022) (width 0.2) (layer "B.Cu") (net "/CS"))
 (segment (start 131.055978 115.139899) (end 130.235877 115.96) (width 0.2) (layer "B.Cu") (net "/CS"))
 (segment (start 130.235877 115.96) (end 129.076079 115.96) (width 0.2) (layer "B.Cu") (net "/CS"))
 (segment (start 128.255978 115.139899) (end 128.255978 108.321663) (width 0.2) (layer "B.Cu") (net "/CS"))
 (segment (start 128.255978 108.321663) (end 125.484315 105.55) (width 0.2) (layer "B.Cu") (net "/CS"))
 (segment (start 113.505978 106.8) (end 110.305978 103.6) (width 0.2) (layer "B.Cu") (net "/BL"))
 (segment (start 150.102989 104.9385) (end 136.69287 104.9385) (width 0.2) (layer "B.Cu") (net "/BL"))
 (segment (start 131.455978 110.175392) (end 131.455978 115.727056) (width 0.2) (layer "B.Cu") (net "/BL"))
 (segment (start 127.185978 107.817349) (end 126.168629 106.8) (width 0.2) (layer "B.Cu") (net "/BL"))
 (segment (start 127.185978 117.597056) (end 127.185978 107.817349) (width 0.2) (layer "B.Cu") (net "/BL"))
 (segment (start 127.888922 118.3) (end 127.185978 117.597056) (width 0.2) (layer "B.Cu") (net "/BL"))
 (segment (start 126.168629 106.8) (end 113.505978 106.8) (width 0.2) (layer "B.Cu") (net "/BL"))
 (segment (start 136.69287 104.9385) (end 131.455978 110.175392) (width 0.2) (layer "B.Cu") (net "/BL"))
 (segment (start 131.455978 115.727056) (end 128.883034 118.3) (width 0.2) (layer "B.Cu") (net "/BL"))
 (segment (start 128.883034 118.3) (end 127.888922 118.3) (width 0.2) (layer "B.Cu") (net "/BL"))
 (segment (start 134.862989 99.8585) (end 133.575814 99.8585) (width 0.2) (layer "B.Cu") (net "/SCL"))
 (segment (start 129.255978 104.178337) (end 129.255978 104.73) (width 0.2) (layer "B.Cu") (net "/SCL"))
 (segment (start 133.575814 99.8585) (end 129.255978 104.178337) (width 0.2) (layer "B.Cu") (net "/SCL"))
 (segment (start 129.255978 104.73) (end 128.835978 105.15) (width 0.2) (layer "B.Cu") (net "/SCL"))
 (segment (start 128.835978 105.15) (end 122.015978 105.15) (width 0.2) (layer "B.Cu") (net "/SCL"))
 (segment (start 122.015978 105.15) (end 120.465978 103.6) (width 0.2) (layer "B.Cu") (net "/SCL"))
 (segment (start 134.862989 97.3185) (end 135.924989 98.3805) (width 0.2) (layer "F.Cu") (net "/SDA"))
 (segment (start 135.924989 98.3805) (end 135.924989 100.298395) (width 0.2) (layer "F.Cu") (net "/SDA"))
 (segment (start 135.302884 100.9205) (end 125.685478 100.9205) (width 0.2) (layer "F.Cu") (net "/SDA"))
 (segment (start 135.924989 100.298395) (end 135.302884 100.9205) (width 0.2) (layer "F.Cu") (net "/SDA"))
 (segment (start 125.685478 100.9205) (end 123.005978 103.6) (width 0.2) (layer "F.Cu") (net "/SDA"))
 (segment (start 129.287478 97.3185) (end 123.005978 103.6) (width 0.2) (layer "B.Cu") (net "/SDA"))
 (segment (start 134.027989 97.3185) (end 129.287478 97.3185) (width 0.2) (layer "B.Cu") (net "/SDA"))
 (segment (start 129.655814 94.7785) (end 121.855978 102.578336) (width 0.2) (layer "B.Cu") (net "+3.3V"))
 (segment (start 122.529632 104.75) (end 124.395978 104.75) (width 0.2) (layer "B.Cu") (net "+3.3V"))
 (segment (start 121.855978 104.076346) (end 122.529632 104.75) (width 0.2) (layer "B.Cu") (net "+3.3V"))
 (segment (start 134.862989 94.7785) (end 129.655814 94.7785) (width 0.2) (layer "B.Cu") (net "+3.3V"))
 (segment (start 124.395978 104.75) (end 125.545978 103.6) (width 0.2) (layer "B.Cu") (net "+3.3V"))
 (segment (start 121.855978 102.578336) (end 121.855978 104.076346) (width 0.2) (layer "B.Cu") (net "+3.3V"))
 (segment (start 134.6985 89.6985) (end 134.5 89.5) (width 0.2) (layer "F.Cu") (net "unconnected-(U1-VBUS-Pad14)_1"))
 (segment (start 134.862989 89.6985) (end 134.6985 89.6985) (width 0.2) (layer "F.Cu") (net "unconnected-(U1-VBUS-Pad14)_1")))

